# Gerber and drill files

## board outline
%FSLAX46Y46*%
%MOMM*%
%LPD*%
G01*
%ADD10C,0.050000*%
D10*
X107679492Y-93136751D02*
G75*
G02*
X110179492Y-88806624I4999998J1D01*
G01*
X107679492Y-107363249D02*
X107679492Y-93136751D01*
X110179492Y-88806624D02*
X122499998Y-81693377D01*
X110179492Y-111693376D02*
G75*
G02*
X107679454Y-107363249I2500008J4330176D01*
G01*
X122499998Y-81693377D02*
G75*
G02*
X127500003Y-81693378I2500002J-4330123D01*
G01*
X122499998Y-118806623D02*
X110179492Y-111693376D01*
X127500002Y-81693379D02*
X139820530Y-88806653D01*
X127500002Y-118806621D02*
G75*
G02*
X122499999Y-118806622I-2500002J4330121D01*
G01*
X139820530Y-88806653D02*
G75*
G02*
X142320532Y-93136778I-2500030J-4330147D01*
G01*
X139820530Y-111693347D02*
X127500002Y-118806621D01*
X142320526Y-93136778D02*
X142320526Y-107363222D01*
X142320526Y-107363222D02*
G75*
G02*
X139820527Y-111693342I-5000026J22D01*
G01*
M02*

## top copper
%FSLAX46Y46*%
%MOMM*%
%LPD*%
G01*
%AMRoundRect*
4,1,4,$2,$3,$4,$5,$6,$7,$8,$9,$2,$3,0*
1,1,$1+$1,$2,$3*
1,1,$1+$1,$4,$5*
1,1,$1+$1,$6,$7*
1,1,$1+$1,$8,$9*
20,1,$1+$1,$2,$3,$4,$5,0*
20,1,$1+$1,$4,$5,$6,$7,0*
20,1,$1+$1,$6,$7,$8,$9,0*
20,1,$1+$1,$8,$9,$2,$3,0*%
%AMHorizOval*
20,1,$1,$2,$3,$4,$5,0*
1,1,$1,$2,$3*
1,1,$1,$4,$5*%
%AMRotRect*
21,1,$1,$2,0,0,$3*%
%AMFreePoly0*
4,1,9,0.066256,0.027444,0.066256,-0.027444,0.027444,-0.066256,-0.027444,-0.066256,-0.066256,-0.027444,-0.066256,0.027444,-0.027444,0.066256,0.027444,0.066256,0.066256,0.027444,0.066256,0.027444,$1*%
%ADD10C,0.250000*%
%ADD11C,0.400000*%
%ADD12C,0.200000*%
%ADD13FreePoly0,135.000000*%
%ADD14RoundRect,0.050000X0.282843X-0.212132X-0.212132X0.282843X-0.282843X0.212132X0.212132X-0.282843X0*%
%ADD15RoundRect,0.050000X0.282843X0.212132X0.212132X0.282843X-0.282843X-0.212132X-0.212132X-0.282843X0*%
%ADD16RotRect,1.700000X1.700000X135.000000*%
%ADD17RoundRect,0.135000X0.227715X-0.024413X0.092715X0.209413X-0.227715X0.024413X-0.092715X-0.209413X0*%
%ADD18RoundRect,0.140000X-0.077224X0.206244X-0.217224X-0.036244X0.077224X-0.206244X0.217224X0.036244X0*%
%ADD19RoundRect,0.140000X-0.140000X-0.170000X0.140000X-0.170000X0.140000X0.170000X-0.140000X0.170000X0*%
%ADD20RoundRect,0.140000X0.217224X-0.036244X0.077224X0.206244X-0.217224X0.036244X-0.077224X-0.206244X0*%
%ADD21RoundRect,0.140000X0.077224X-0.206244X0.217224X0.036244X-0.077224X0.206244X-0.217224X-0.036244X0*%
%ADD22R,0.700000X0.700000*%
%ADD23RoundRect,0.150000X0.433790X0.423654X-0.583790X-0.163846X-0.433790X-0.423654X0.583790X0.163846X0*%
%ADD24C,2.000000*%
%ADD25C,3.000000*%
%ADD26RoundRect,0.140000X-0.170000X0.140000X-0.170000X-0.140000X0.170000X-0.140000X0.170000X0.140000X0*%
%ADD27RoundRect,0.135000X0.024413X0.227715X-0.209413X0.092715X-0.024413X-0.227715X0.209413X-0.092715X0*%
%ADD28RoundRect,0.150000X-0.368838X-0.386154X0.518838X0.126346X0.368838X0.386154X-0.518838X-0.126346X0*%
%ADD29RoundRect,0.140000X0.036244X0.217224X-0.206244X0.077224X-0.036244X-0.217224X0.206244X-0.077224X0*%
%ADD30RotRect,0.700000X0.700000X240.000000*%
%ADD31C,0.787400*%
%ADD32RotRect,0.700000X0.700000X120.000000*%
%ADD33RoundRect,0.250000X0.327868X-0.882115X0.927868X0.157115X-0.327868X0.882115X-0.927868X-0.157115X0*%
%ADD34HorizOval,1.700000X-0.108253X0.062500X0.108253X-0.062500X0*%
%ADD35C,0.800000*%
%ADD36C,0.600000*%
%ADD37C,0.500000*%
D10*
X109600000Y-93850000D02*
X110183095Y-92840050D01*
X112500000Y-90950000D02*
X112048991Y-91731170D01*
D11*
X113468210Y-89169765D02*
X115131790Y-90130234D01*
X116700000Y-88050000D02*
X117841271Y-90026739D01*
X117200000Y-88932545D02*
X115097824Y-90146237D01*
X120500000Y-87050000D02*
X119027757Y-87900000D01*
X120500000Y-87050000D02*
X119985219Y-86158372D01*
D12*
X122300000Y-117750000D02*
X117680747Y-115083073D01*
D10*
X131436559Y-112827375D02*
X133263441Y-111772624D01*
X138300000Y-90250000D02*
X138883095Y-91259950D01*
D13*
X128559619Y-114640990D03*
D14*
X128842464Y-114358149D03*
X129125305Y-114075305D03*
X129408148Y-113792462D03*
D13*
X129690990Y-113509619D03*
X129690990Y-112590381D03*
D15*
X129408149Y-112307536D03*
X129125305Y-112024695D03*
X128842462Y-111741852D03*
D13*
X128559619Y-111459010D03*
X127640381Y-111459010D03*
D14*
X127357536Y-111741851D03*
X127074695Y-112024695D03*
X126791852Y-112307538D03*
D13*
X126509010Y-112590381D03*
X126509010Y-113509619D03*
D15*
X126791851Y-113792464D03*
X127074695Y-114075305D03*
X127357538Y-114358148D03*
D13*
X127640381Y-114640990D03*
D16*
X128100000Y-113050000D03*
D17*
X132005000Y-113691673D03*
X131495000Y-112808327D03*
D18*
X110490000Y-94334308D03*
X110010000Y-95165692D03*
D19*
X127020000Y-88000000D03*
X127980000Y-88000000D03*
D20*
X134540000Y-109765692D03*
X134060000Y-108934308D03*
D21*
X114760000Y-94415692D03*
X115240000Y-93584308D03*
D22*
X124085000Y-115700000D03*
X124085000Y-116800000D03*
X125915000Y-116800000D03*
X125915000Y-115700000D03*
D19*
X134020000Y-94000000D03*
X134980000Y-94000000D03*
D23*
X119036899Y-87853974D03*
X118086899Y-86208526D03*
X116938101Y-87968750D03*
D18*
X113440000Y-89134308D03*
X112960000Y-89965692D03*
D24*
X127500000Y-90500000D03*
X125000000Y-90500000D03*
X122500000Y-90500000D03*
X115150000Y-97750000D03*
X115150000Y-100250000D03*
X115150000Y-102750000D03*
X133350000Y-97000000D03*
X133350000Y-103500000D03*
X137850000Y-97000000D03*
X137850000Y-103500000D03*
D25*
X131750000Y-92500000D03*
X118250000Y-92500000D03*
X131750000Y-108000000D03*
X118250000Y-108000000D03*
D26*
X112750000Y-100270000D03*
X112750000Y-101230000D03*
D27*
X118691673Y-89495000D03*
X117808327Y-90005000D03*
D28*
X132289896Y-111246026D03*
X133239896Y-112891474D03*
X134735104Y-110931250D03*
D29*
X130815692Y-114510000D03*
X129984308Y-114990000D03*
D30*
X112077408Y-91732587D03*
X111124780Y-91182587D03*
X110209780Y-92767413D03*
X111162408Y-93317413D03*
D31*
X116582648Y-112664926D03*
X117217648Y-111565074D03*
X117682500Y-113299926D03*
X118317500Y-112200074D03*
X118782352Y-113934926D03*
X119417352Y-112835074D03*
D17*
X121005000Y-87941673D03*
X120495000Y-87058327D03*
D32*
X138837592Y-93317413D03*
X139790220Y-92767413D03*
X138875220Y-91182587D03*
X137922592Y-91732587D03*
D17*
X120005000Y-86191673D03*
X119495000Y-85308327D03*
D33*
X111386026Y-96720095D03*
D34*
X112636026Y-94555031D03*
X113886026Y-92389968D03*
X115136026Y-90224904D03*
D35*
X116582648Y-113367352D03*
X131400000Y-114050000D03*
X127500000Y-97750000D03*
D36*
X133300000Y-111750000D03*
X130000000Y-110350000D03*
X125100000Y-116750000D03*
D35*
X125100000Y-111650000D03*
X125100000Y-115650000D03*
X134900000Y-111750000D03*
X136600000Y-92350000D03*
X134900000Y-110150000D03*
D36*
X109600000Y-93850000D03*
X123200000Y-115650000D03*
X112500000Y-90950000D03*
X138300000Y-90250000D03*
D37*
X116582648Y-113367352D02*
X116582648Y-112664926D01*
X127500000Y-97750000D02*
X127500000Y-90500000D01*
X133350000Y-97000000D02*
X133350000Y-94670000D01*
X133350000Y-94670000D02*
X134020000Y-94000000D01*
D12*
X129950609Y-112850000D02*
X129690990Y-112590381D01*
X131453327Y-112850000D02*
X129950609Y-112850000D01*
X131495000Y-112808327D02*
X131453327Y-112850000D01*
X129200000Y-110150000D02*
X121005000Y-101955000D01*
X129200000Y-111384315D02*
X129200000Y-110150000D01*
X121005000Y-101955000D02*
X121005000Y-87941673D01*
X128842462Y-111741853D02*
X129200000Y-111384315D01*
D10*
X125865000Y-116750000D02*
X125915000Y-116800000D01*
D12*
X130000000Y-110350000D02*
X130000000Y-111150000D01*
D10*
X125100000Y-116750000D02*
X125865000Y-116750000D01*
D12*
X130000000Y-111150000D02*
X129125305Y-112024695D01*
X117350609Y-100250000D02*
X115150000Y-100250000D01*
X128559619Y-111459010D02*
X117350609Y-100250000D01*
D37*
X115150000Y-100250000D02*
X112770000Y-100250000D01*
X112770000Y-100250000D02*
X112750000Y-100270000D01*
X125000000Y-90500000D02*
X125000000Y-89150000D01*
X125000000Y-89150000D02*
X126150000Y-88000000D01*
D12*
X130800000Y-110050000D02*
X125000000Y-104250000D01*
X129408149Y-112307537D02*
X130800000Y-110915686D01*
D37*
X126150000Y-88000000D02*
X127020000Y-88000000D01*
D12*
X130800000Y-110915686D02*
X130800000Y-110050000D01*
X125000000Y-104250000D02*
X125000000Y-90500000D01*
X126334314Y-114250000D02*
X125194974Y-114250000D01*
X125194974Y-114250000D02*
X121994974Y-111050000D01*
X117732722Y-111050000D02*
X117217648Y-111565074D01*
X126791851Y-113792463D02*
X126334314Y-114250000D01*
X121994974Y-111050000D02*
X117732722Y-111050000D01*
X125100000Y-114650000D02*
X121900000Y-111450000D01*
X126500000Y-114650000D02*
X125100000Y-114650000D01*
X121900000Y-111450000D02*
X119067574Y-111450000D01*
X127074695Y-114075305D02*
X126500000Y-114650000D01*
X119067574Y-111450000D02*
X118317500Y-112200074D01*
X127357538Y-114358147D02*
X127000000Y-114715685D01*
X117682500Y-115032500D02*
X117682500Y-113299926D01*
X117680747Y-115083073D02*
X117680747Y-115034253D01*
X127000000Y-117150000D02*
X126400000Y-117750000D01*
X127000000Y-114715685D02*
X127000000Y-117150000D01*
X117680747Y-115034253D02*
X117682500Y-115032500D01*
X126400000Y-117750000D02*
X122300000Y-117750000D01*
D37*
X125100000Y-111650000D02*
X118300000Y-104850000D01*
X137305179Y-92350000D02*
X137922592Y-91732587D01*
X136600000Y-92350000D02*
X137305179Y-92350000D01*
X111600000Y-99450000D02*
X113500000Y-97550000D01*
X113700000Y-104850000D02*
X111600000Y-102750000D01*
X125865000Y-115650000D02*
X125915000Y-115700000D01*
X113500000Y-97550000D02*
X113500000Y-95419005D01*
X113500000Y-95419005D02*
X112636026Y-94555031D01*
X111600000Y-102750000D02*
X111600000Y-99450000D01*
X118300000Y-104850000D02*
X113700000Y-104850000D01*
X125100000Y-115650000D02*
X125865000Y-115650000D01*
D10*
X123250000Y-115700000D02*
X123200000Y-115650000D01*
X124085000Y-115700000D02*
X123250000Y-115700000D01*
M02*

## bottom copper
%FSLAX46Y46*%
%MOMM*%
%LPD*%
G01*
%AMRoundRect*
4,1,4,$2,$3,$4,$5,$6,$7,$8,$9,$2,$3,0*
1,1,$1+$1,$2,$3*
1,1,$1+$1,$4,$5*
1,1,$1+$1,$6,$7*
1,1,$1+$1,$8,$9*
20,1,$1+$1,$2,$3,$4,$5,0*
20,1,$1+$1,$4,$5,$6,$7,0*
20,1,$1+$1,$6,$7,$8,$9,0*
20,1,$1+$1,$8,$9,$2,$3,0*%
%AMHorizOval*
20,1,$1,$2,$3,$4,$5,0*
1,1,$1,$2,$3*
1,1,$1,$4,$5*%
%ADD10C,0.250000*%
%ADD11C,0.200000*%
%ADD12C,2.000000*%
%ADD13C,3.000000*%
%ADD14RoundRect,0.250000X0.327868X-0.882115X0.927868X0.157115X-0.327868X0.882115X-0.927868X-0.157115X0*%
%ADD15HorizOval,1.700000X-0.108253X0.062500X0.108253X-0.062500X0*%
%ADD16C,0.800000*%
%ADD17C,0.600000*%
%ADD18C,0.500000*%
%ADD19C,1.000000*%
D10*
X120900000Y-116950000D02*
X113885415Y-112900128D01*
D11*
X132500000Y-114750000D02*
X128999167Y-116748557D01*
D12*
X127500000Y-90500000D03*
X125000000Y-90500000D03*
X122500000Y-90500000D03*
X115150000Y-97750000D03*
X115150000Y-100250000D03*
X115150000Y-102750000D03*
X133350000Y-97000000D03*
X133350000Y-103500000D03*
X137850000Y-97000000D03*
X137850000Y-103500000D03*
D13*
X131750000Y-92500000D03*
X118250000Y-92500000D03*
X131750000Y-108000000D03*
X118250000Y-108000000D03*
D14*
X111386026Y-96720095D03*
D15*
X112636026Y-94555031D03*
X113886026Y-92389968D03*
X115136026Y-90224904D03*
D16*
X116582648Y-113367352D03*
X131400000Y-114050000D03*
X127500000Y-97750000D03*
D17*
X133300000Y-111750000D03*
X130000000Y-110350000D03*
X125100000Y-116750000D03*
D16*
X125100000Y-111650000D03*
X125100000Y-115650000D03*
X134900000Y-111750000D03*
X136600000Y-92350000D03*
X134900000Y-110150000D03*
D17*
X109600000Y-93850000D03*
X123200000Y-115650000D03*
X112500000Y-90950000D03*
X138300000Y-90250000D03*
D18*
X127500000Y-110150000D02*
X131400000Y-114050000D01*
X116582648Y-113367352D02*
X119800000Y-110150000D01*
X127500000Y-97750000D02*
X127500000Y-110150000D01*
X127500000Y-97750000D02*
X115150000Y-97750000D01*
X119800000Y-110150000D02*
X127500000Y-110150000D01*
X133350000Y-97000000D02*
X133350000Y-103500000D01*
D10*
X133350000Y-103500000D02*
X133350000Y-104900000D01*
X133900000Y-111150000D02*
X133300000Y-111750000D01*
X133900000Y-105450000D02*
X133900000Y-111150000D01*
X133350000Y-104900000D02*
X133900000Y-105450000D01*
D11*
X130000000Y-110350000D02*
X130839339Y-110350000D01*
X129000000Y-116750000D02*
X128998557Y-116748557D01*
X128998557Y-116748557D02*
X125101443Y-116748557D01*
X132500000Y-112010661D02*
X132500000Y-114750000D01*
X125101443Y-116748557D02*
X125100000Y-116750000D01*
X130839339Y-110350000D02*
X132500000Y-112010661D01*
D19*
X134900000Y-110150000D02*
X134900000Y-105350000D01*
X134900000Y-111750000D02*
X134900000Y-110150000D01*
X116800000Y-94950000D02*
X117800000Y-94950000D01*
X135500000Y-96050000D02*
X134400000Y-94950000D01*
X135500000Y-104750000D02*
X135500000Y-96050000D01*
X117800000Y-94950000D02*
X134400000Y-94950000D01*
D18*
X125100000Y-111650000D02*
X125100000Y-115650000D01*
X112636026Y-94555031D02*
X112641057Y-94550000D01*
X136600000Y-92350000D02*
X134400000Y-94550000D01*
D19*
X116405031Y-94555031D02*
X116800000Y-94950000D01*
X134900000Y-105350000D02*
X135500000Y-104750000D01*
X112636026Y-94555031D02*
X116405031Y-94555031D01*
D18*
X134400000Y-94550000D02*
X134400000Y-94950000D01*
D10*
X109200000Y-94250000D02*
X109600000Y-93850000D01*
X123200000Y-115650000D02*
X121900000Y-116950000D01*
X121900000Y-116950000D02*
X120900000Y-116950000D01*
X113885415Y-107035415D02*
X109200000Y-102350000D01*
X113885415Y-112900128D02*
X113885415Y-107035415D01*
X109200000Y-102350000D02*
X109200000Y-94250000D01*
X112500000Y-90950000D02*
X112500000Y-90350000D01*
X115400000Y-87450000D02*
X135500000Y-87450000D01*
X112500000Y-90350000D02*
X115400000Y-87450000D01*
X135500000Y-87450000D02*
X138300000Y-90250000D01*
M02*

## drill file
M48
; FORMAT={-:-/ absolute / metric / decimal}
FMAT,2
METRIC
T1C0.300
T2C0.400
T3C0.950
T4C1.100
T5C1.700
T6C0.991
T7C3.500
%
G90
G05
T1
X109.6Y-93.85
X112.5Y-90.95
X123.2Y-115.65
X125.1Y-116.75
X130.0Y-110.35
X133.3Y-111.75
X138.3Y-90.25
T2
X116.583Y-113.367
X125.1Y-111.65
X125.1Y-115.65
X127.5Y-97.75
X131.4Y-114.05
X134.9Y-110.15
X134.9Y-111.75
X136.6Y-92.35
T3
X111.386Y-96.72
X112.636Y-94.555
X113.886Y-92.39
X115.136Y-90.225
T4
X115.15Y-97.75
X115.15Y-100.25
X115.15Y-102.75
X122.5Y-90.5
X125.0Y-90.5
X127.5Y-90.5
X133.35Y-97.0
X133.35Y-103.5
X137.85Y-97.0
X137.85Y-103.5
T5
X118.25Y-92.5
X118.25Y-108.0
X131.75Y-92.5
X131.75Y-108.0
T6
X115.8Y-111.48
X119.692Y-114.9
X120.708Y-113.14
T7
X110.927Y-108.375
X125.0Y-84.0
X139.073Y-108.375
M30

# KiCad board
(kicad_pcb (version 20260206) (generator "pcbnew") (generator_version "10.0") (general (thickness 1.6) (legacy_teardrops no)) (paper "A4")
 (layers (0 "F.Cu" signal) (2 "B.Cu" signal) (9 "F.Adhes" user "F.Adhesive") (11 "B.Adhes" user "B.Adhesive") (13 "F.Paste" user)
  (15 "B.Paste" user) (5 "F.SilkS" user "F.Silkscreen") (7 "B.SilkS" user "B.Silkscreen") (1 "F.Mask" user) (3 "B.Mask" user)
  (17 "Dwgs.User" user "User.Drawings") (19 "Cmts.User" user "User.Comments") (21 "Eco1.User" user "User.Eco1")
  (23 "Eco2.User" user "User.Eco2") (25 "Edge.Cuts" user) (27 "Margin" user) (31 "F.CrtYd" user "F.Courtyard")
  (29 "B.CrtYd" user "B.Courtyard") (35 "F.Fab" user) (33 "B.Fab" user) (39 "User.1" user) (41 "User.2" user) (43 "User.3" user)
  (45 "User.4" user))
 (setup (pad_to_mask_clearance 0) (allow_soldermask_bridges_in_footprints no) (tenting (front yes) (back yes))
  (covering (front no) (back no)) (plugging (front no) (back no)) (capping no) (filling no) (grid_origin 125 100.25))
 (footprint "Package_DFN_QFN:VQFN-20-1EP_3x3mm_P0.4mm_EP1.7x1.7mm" (layer "F.Cu") (at 128.1 113.05 135)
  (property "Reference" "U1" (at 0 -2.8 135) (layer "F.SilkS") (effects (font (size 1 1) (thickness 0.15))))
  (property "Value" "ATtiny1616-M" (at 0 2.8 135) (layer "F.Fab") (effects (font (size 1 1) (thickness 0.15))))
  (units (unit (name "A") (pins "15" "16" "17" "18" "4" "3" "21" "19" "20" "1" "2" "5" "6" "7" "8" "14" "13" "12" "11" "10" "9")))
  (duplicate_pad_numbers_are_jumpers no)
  (pad "" smd roundrect (at -0.425 -0.425 135) (size 0.69 0.69) (layers "F.Paste") (roundrect_rratio 0.25))
  (pad "" smd roundrect (at -0.425 0.425 135) (size 0.69 0.69) (layers "F.Paste") (roundrect_rratio 0.25))
  (pad "" smd roundrect (at 0.425 -0.425 135) (size 0.69 0.69) (layers "F.Paste") (roundrect_rratio 0.25))
  (pad "" smd roundrect (at 0.425 0.425 135) (size 0.69 0.69) (layers "F.Paste") (roundrect_rratio 0.25))
  (pad "1" smd custom (at -1.45 -0.8 135) (size 0.143431 0.143431) (layers "F.Cu" "F.Mask" "F.Paste") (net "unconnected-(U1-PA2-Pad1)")
   (options (clearance outline) (anchor circle)) (primitives))
  (pad "2" smd roundrect (at -1.450002 -0.4 135) (size 0.8 0.2) (layers "F.Cu" "F.Mask" "F.Paste") (roundrect_rratio 0.25)
   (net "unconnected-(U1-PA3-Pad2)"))
  (pad "3" smd roundrect (at -1.45 0 135) (size 0.8 0.2) (layers "F.Cu" "F.Mask" "F.Paste") (roundrect_rratio 0.25) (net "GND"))
  (pad "4" smd roundrect (at -1.45 0.4 135) (size 0.8 0.2) (layers "F.Cu" "F.Mask" "F.Paste") (roundrect_rratio 0.25) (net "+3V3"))
  (pad "5" smd custom (at -1.45 0.8 135) (size 0.143431 0.143431) (layers "F.Cu" "F.Mask" "F.Paste") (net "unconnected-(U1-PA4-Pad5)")
   (options (clearance outline) (anchor circle)) (primitives))
  (pad "6" smd custom (at -0.8 1.45 135) (size 0.143431 0.143431) (layers "F.Cu" "F.Mask" "F.Paste") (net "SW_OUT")
   (options (clearance outline) (anchor circle)) (primitives))
  (pad "7" smd roundrect (at -0.4 1.450002 135) (size 0.2 0.8) (layers "F.Cu" "F.Mask" "F.Paste") (roundrect_rratio 0.25) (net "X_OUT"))
  (pad "8" smd roundrect (at 0 1.45 135) (size 0.2 0.8) (layers "F.Cu" "F.Mask" "F.Paste") (roundrect_rratio 0.25) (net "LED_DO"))
  (pad "9" smd roundrect (at 0.4 1.45 135) (size 0.2 0.8) (layers "F.Cu" "F.Mask" "F.Paste") (roundrect_rratio 0.25) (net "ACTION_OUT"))
  (pad "10" smd custom (at 0.8 1.45 135) (size 0.143431 0.143431) (layers "F.Cu" "F.Mask" "F.Paste") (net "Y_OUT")
   (options (clearance outline) (anchor circle)) (primitives))
  (pad "11" smd custom (at 1.45 0.8 135) (size 0.143431 0.143431) (layers "F.Cu" "F.Mask" "F.Paste") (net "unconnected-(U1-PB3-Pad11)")
   (options (clearance outline) (anchor circle)) (primitives))
  (pad "12" smd roundrect (at 1.450002 0.4 135) (size 0.8 0.2) (layers "F.Cu" "F.Mask" "F.Paste") (roundrect_rratio 0.25)
   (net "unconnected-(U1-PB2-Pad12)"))
  (pad "13" smd roundrect (at 1.45 0 135) (size 0.8 0.2) (layers "F.Cu" "F.Mask" "F.Paste") (roundrect_rratio 0.25)
   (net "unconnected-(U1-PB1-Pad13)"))
  (pad "14" smd roundrect (at 1.45 -0.4 135) (size 0.8 0.2) (layers "F.Cu" "F.Mask" "F.Paste") (roundrect_rratio 0.25)
   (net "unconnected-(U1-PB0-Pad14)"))
  (pad "15" smd custom (at 1.45 -0.8 135) (size 0.143431 0.143431) (layers "F.Cu" "F.Mask" "F.Paste") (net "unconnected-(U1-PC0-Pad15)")
   (options (clearance outline) (anchor circle)) (primitives))
  (pad "16" smd custom (at 0.8 -1.45 135) (size 0.143431 0.143431) (layers "F.Cu" "F.Mask" "F.Paste") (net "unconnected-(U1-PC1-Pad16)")
   (options (clearance outline) (anchor circle)) (primitives))
  (pad "17" smd roundrect (at 0.4 -1.450002 135) (size 0.2 0.8) (layers "F.Cu" "F.Mask" "F.Paste") (roundrect_rratio 0.25) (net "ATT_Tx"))
  (pad "18" smd roundrect (at 0 -1.45 135) (size 0.2 0.8) (layers "F.Cu" "F.Mask" "F.Paste") (roundrect_rratio 0.25) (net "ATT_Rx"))
  (pad "19" smd roundrect (at -0.4 -1.45 135) (size 0.2 0.8) (layers "F.Cu" "F.Mask" "F.Paste") (roundrect_rratio 0.25) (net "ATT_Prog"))
  (pad "20" smd custom (at -0.8 -1.45 135) (size 0.143431 0.143431) (layers "F.Cu" "F.Mask" "F.Paste") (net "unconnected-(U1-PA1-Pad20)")
   (options (clearance outline) (anchor circle)) (primitives))
  (pad "21" smd rect (at 0 0 135) (size 1.7 1.7) (layers "F.Cu" "F.Mask") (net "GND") (zone_connect 2)))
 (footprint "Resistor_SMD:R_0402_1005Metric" (layer "F.Cu") (at 131.75 113.25 120)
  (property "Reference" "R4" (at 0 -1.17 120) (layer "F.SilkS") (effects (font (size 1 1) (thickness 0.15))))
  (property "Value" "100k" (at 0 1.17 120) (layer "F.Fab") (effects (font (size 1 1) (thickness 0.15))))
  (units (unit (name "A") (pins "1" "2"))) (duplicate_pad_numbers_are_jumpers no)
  (pad "1" smd roundrect (at -0.51 0 120) (size 0.54 0.64) (layers "F.Cu" "F.Mask" "F.Paste") (roundrect_rratio 0.25) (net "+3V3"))
  (pad "2" smd roundrect (at 0.51 0 120) (size 0.54 0.64) (layers "F.Cu" "F.Mask" "F.Paste") (roundrect_rratio 0.25) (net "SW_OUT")))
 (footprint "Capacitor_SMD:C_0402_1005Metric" (layer "F.Cu") (at 110.25 94.75 -120)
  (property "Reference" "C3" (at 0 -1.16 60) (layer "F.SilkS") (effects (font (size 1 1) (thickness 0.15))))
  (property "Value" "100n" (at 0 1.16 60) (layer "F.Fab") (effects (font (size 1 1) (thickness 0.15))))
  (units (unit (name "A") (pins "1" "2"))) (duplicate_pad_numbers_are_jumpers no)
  (pad "1" smd roundrect (at -0.48 0 240) (size 0.56 0.62) (layers "F.Cu" "F.Mask" "F.Paste") (roundrect_rratio 0.25) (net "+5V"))
  (pad "2" smd roundrect (at 0.48 0 240) (size 0.56 0.62) (layers "F.Cu" "F.Mask" "F.Paste") (roundrect_rratio 0.25) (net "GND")))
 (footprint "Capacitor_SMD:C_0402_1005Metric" (layer "F.Cu") (at 127.5 88)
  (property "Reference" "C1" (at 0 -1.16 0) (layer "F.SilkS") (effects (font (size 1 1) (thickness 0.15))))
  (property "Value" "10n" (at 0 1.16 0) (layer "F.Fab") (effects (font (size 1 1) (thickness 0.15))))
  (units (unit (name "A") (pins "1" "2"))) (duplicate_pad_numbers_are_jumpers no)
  (pad "1" smd roundrect (at -0.48 0) (size 0.56 0.62) (layers "F.Cu" "F.Mask" "F.Paste") (roundrect_rratio 0.25) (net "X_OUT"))
  (pad "2" smd roundrect (at 0.48 0) (size 0.56 0.62) (layers "F.Cu" "F.Mask" "F.Paste") (roundrect_rratio 0.25) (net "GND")))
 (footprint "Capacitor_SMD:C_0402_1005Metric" (layer "F.Cu") (at 134.3 109.35 120)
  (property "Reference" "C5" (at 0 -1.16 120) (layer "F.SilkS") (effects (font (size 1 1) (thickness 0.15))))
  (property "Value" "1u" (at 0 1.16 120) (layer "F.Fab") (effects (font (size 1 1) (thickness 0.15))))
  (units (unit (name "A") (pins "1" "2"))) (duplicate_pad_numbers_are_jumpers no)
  (pad "1" smd roundrect (at -0.48 0 120) (size 0.56 0.62) (layers "F.Cu" "F.Mask" "F.Paste") (roundrect_rratio 0.25) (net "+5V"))
  (pad "2" smd roundrect (at 0.48 0 120) (size 0.56 0.62) (layers "F.Cu" "F.Mask" "F.Paste") (roundrect_rratio 0.25) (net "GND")))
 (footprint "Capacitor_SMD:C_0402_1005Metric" (layer "F.Cu") (at 115 94 60)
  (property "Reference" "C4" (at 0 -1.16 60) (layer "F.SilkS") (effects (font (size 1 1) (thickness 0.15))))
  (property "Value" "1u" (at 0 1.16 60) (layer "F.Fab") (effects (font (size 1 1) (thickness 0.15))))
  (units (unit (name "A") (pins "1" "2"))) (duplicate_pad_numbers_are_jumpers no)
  (pad "1" smd roundrect (at -0.48 0 60) (size 0.56 0.62) (layers "F.Cu" "F.Mask" "F.Paste") (roundrect_rratio 0.25) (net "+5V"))
  (pad "2" smd roundrect (at 0.48 0 60) (size 0.56 0.62) (layers "F.Cu" "F.Mask" "F.Paste") (roundrect_rratio 0.25) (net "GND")))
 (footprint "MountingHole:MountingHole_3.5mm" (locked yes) (layer "F.Cu") (at 110.927087 108.375)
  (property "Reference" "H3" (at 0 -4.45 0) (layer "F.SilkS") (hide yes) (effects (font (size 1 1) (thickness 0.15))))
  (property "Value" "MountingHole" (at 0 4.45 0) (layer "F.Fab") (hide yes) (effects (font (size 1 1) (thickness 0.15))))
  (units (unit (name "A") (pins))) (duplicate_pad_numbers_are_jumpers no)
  (pad "" np_thru_hole circle (at 0 0) (size 3.5 3.5) (drill 3.5) (layers "*.Cu" "*.Mask")))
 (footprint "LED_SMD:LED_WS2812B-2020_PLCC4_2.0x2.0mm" (layer "F.Cu") (at 125 116.25)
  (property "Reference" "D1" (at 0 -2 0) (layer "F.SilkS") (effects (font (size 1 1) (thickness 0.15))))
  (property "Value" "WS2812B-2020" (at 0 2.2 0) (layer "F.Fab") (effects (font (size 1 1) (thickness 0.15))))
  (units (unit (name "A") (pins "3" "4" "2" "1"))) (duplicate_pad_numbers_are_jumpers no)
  (pad "1" smd rect (at -0.915 -0.55) (size 0.7 0.7) (layers "F.Cu" "F.Mask" "F.Paste") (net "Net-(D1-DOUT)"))
  (pad "2" smd rect (at -0.915 0.55) (size 0.7 0.7) (layers "F.Cu" "F.Mask" "F.Paste") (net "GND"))
  (pad "3" smd rect (at 0.915 0.55) (size 0.7 0.7) (layers "F.Cu" "F.Mask" "F.Paste") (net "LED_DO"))
  (pad "4" smd rect (at 0.915 -0.55) (size 0.7 0.7) (layers "F.Cu" "F.Mask" "F.Paste") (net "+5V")))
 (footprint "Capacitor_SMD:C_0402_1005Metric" (layer "F.Cu") (at 134.5 94)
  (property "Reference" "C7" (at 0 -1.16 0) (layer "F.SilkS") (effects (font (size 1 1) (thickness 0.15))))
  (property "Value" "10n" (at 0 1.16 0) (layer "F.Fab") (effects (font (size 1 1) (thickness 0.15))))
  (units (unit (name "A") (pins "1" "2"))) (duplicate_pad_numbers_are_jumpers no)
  (pad "1" smd roundrect (at -0.48 0) (size 0.56 0.62) (layers "F.Cu" "F.Mask" "F.Paste") (roundrect_rratio 0.25) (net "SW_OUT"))
  (pad "2" smd roundrect (at 0.48 0) (size 0.56 0.62) (layers "F.Cu" "F.Mask" "F.Paste") (roundrect_rratio 0.25) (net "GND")))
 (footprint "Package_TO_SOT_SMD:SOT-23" (layer "F.Cu") (at 117.75 87.5 -150)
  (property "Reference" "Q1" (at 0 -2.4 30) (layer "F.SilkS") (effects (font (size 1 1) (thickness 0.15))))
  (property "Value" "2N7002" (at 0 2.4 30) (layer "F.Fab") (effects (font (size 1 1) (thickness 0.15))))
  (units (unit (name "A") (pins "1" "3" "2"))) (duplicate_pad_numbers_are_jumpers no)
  (pad "1" smd roundrect (at -0.9375 -0.95 210) (size 1.475 0.6) (layers "F.Cu" "F.Mask" "F.Paste") (roundrect_rratio 0.25)
   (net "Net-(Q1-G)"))
  (pad "2" smd roundrect (at -0.9375 0.95 210) (size 1.475 0.6) (layers "F.Cu" "F.Mask" "F.Paste") (roundrect_rratio 0.25) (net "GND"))
  (pad "3" smd roundrect (at 0.9375 0 210) (size 1.475 0.6) (layers "F.Cu" "F.Mask" "F.Paste") (roundrect_rratio 0.25) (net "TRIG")))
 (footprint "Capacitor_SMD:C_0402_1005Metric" (layer "F.Cu") (at 113.2 89.55 -120)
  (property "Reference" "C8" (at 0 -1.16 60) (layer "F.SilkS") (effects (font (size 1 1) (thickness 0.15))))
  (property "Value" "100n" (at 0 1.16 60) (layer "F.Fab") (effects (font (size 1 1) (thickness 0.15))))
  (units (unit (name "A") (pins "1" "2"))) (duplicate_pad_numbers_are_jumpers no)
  (pad "1" smd roundrect (at -0.48 0 240) (size 0.56 0.62) (layers "F.Cu" "F.Mask" "F.Paste") (roundrect_rratio 0.25) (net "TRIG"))
  (pad "2" smd roundrect (at 0.48 0 240) (size 0.56 0.62) (layers "F.Cu" "F.Mask" "F.Paste") (roundrect_rratio 0.25) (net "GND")))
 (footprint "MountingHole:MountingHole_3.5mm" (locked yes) (layer "F.Cu") (at 125 84)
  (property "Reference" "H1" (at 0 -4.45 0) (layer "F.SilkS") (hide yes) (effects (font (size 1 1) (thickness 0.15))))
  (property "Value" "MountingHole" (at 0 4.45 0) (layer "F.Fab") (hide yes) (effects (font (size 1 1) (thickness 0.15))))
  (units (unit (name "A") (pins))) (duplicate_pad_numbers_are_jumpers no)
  (pad "" np_thru_hole circle (at 0 0) (size 3.5 3.5) (drill 3.5) (layers "*.Cu" "*.Mask")))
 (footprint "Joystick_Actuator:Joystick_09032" (layer "F.Cu") (at 125 100.25 -90)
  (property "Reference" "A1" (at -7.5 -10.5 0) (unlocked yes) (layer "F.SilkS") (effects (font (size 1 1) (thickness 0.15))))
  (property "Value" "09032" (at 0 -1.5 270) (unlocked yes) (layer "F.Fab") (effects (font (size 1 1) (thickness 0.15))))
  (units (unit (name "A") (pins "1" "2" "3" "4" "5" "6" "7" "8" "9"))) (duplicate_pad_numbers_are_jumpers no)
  (pad "1" thru_hole circle (at -9.75 -2.5 270) (size 2 2) (drill 1.1) (layers "*.Cu" "*.Mask") (remove_unused_layers no) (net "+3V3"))
  (pad "2" thru_hole circle (at -9.75 0 270) (size 2 2) (drill 1.1) (layers "*.Cu" "*.Mask") (remove_unused_layers no) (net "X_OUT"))
  (pad "3" thru_hole circle (at -9.75 2.5 270) (size 2 2) (drill 1.1) (layers "*.Cu" "*.Mask") (remove_unused_layers no) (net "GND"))
  (pad "4" thru_hole circle (at -2.5 9.85 270) (size 2 2) (drill 1.1) (layers "*.Cu" "*.Mask") (remove_unused_layers no) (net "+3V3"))
  (pad "5" thru_hole circle (at 0 9.85 270) (size 2 2) (drill 1.1) (layers "*.Cu" "*.Mask") (remove_unused_layers no) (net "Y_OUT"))
  (pad "6" thru_hole circle (at 2.5 9.85 270) (size 2 2) (drill 1.1) (layers "*.Cu" "*.Mask") (remove_unused_layers no) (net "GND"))
  (pad "7" thru_hole circle (at -3.25 -8.35 270) (size 2 2) (drill 1.1) (layers "*.Cu" "*.Mask") (remove_unused_layers no) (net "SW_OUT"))
  (pad "7" thru_hole circle (at 3.25 -8.35 270) (size 2 2) (drill 1.1) (layers "*.Cu" "*.Mask") (remove_unused_layers no) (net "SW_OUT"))
  (pad "8" thru_hole circle (at -3.25 -12.85 270) (size 2 2) (drill 1.1) (layers "*.Cu" "*.Mask") (remove_unused_layers no) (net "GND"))
  (pad "8" thru_hole circle (at 3.25 -12.85 270) (size 2 2) (drill 1.1) (layers "*.Cu" "*.Mask") (remove_unused_layers no) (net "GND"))
  (pad "9" thru_hole circle (at -7.75 -6.75 270) (size 3 3) (drill 1.7) (layers "*.Cu" "*.Mask") (remove_unused_layers no) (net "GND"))
  (pad "9" thru_hole circle (at -7.75 6.75 270) (size 3 3) (drill 1.7) (layers "*.Cu" "*.Mask") (remove_unused_layers no) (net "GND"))
  (pad "9" thru_hole circle (at 7.75 -6.75 270) (size 3 3) (drill 1.7) (layers "*.Cu" "*.Mask") (remove_unused_layers no) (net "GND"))
  (pad "9" thru_hole circle (at 7.75 6.75 270) (size 3 3) (drill 1.7) (layers "*.Cu" "*.Mask") (remove_unused_layers no) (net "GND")))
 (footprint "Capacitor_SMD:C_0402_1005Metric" (layer "F.Cu") (at 112.75 100.75 -90)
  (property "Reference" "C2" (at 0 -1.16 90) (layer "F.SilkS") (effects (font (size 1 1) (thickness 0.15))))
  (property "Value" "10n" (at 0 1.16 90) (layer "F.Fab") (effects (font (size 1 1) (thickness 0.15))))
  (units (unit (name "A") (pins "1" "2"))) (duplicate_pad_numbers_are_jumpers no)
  (pad "1" smd roundrect (at -0.48 0 270) (size 0.56 0.62) (layers "F.Cu" "F.Mask" "F.Paste") (roundrect_rratio 0.25) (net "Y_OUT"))
  (pad "2" smd roundrect (at 0.48 0 270) (size 0.56 0.62) (layers "F.Cu" "F.Mask" "F.Paste") (roundrect_rratio 0.25) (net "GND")))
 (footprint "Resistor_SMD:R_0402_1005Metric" (layer "F.Cu") (at 118.25 89.75 -150)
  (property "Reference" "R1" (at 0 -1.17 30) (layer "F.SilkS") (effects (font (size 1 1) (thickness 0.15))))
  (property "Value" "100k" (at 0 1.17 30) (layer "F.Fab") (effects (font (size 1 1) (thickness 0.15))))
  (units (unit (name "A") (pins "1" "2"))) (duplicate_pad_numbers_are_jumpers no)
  (pad "1" smd roundrect (at -0.51 0 210) (size 0.54 0.64) (layers "F.Cu" "F.Mask" "F.Paste") (roundrect_rratio 0.25) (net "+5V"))
  (pad "2" smd roundrect (at 0.51 0 210) (size 0.54 0.64) (layers "F.Cu" "F.Mask" "F.Paste") (roundrect_rratio 0.25) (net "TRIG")))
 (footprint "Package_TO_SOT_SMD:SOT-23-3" (layer "F.Cu") (at 133.75 111.5 30)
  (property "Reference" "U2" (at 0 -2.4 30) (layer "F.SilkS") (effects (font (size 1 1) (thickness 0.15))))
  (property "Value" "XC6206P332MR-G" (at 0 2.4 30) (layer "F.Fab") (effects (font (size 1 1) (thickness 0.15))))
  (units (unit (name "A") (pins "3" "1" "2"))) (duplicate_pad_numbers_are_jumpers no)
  (pad "1" smd roundrect (at -1.1375 -0.95 30) (size 1.325 0.6) (layers "F.Cu" "F.Mask" "F.Paste") (roundrect_rratio 0.25) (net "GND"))
  (pad "2" smd roundrect (at -1.1375 0.95 30) (size 1.325 0.6) (layers "F.Cu" "F.Mask" "F.Paste") (roundrect_rratio 0.25) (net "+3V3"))
  (pad "3" smd roundrect (at 1.1375 0 30) (size 1.325 0.6) (layers "F.Cu" "F.Mask" "F.Paste") (roundrect_rratio 0.25) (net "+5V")))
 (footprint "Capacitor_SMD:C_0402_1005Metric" (layer "F.Cu") (at 130.4 114.75 -150)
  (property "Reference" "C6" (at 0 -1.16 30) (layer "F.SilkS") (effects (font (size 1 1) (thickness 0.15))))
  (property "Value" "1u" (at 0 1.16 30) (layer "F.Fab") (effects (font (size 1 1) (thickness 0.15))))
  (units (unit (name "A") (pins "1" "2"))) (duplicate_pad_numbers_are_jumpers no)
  (pad "1" smd roundrect (at -0.48 0 210) (size 0.56 0.62) (layers "F.Cu" "F.Mask" "F.Paste") (roundrect_rratio 0.25) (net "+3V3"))
  (pad "2" smd roundrect (at 0.48 0 210) (size 0.56 0.62) (layers "F.Cu" "F.Mask" "F.Paste") (roundrect_rratio 0.25) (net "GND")))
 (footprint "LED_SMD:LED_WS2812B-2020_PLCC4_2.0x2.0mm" (layer "F.Cu") (at 111.143594 92.25 -120)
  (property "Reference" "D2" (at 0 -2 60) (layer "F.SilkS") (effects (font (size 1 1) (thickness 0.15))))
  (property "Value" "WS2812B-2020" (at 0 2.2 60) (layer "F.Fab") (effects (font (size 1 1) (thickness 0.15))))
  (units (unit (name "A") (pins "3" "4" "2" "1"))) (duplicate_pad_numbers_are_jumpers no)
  (pad "1" smd rect (at -0.915 -0.55 240) (size 0.7 0.7) (layers "F.Cu" "F.Mask" "F.Paste") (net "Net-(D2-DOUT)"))
  (pad "2" smd rect (at -0.915 0.55 240) (size 0.7 0.7) (layers "F.Cu" "F.Mask" "F.Paste") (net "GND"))
  (pad "3" smd rect (at 0.915 0.55 240) (size 0.7 0.7) (layers "F.Cu" "F.Mask" "F.Paste") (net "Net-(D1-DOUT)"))
  (pad "4" smd rect (at 0.915 -0.55 240) (size 0.7 0.7) (layers "F.Cu" "F.Mask" "F.Paste") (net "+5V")))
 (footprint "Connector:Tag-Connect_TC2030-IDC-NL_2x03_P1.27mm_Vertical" (layer "F.Cu") (at 118 112.75 -30)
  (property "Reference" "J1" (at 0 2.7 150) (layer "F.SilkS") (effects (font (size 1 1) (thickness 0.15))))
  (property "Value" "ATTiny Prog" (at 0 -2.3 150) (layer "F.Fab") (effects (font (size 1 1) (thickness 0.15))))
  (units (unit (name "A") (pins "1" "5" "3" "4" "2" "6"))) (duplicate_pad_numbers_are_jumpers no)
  (pad "" np_thru_hole circle (at -2.54 0 330) (size 0.9906 0.9906) (drill 0.9906) (layers "*.Cu" "*.Mask"))
  (pad "" np_thru_hole circle (at 2.540001 -1.016 330) (size 0.9906 0.9906) (drill 0.9906) (layers "*.Cu" "*.Mask"))
  (pad "" np_thru_hole circle (at 2.540001 1.016 330) (size 0.9906 0.9906) (drill 0.9906) (layers "*.Cu" "*.Mask"))
  (pad "1" connect circle (at -1.27 0.635 330) (size 0.7874 0.7874) (layers "F.Cu" "F.Mask") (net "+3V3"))
  (pad "2" connect circle (at -1.27 -0.635 330) (size 0.7874 0.7874) (layers "F.Cu" "F.Mask") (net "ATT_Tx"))
  (pad "3" connect circle (at 0 0.635 330) (size 0.7874 0.7874) (layers "F.Cu" "F.Mask") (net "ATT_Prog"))
  (pad "4" connect circle (at 0 -0.635 330) (size 0.7874 0.7874) (layers "F.Cu" "F.Mask") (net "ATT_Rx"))
  (pad "5" connect circle (at 1.27 0.635 330) (size 0.7874 0.7874) (layers "F.Cu" "F.Mask") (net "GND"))
  (pad "6" connect circle (at 1.27 -0.635 330) (size 0.7874 0.7874) (layers "F.Cu" "F.Mask") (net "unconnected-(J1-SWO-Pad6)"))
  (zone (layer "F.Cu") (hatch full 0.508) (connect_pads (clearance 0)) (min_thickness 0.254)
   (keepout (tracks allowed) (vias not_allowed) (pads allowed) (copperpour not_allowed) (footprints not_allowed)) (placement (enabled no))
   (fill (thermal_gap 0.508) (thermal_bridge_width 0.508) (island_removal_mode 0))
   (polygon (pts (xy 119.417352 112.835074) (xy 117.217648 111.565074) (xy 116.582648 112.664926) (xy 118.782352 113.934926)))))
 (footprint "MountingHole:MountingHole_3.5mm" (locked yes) (layer "F.Cu") (at 139.072913 108.375)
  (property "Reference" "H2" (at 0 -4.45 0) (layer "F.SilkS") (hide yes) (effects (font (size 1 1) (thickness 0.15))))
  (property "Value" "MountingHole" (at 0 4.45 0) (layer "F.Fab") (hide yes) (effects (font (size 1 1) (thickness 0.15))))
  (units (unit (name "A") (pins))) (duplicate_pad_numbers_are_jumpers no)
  (pad "" np_thru_hole circle (at 0 0) (size 3.5 3.5) (drill 3.5) (layers "*.Cu" "*.Mask")))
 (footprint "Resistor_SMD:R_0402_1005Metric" (layer "F.Cu") (at 120.75 87.5 120)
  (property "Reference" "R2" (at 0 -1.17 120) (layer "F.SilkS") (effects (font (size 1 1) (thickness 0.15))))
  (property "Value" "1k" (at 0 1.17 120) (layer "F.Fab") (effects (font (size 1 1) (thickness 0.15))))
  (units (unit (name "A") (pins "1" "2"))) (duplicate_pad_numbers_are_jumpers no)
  (pad "1" smd roundrect (at -0.51 0 120) (size 0.54 0.64) (layers "F.Cu" "F.Mask" "F.Paste") (roundrect_rratio 0.25) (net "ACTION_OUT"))
  (pad "2" smd roundrect (at 0.51 0 120) (size 0.54 0.64) (layers "F.Cu" "F.Mask" "F.Paste") (roundrect_rratio 0.25) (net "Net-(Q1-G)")))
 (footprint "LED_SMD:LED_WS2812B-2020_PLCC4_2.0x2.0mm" (layer "F.Cu") (at 138.856406 92.25 120)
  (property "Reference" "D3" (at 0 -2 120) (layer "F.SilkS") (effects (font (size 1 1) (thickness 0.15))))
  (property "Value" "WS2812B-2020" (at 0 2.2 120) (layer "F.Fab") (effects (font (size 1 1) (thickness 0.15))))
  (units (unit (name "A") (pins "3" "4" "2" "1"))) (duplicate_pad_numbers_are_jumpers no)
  (pad "1" smd rect (at -0.915 -0.55 120) (size 0.7 0.7) (layers "F.Cu" "F.Mask" "F.Paste") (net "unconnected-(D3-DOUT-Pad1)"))
  (pad "2" smd rect (at -0.915 0.55 120) (size 0.7 0.7) (layers "F.Cu" "F.Mask" "F.Paste") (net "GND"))
  (pad "3" smd rect (at 0.915 0.55 120) (size 0.7 0.7) (layers "F.Cu" "F.Mask" "F.Paste") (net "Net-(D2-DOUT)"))
  (pad "4" smd rect (at 0.915 -0.55 120) (size 0.7 0.7) (layers "F.Cu" "F.Mask" "F.Paste") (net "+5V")))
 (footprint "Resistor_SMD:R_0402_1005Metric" (layer "F.Cu") (at 119.75 85.75 120)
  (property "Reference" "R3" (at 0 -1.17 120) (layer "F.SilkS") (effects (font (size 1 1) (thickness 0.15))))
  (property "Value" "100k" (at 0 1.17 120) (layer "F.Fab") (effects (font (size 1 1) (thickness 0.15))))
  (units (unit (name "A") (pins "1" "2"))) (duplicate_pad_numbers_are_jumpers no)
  (pad "1" smd roundrect (at -0.51 0 120) (size 0.54 0.64) (layers "F.Cu" "F.Mask" "F.Paste") (roundrect_rratio 0.25) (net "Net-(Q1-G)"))
  (pad "2" smd roundrect (at 0.51 0 120) (size 0.54 0.64) (layers "F.Cu" "F.Mask" "F.Paste") (roundrect_rratio 0.25) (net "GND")))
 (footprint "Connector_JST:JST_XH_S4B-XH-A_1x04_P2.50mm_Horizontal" (layer "B.Cu") (at 111.386026 96.720095 60)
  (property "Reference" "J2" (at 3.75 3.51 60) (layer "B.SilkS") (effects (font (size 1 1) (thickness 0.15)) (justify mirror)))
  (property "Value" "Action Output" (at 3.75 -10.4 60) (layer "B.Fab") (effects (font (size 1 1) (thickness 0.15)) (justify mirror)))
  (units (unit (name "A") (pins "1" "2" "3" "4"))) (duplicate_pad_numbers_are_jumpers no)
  (pad "1" thru_hole roundrect (at 0 0 60) (size 1.7 1.95) (drill 0.95) (layers "*.Cu" "*.Mask") (remove_unused_layers no)
   (roundrect_rratio 0.147059) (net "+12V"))
  (pad "2" thru_hole oval (at 2.5 0 60) (size 1.7 1.95) (drill 0.95) (layers "*.Cu" "*.Mask") (remove_unused_layers no) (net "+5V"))
  (pad "3" thru_hole oval (at 5 0 60) (size 1.7 1.95) (drill 0.95) (layers "*.Cu" "*.Mask") (remove_unused_layers no) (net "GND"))
  (pad "4" thru_hole oval (at 7.5 0 60) (size 1.7 1.95) (drill 0.95) (layers "*.Cu" "*.Mask") (remove_unused_layers no) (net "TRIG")))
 (gr_line (start 109.6 93.85) (end 110.183095 92.84005) (stroke (width 0.25) (type solid)) (layer "F.Cu") (net "Net-(D1-DOUT)"))
 (gr_line (start 112.5 90.95) (end 112.048991 91.73117) (stroke (width 0.25) (type solid)) (layer "F.Cu") (net "Net-(D2-DOUT)"))
 (gr_line (start 113.46821 89.169765) (end 115.13179 90.130234) (stroke (width 0.4) (type solid)) (layer "F.Cu") (net "TRIG"))
 (gr_line (start 116.7 88.05) (end 117.841271 90.026739) (stroke (width 0.4) (type solid)) (layer "F.Cu") (net "TRIG"))
 (gr_line (start 117.2 88.932545) (end 115.097824 90.146237) (stroke (width 0.4) (type solid)) (layer "F.Cu") (net "TRIG"))
 (gr_line (start 120.5 87.05) (end 119.027757 87.9) (stroke (width 0.4) (type solid)) (layer "F.Cu") (net "Net-(Q1-G)"))
 (gr_line (start 120.5 87.05) (end 119.985219 86.158372) (stroke (width 0.4) (type solid)) (layer "F.Cu") (net "Net-(Q1-G)"))
 (gr_line (start 122.3 117.75) (end 117.680747 115.083073) (stroke (width 0.2) (type solid)) (layer "F.Cu") (net "ATT_Prog"))
 (gr_line (start 131.436559 112.827375) (end 133.263441 111.772624) (stroke (width 0.25) (type solid)) (layer "F.Cu") (net "SW_OUT"))
 (gr_line (start 138.3 90.25) (end 138.883095 91.25995) (stroke (width 0.25) (type solid)) (layer "F.Cu") (net "Net-(D2-DOUT)"))
 (gr_line (start 120.9 116.95) (end 113.885415 112.900128) (stroke (width 0.25) (type solid)) (layer "B.Cu") (net "Net-(D1-DOUT)"))
 (gr_line (start 132.5 114.75) (end 128.999167 116.748557) (stroke (width 0.2) (type solid)) (layer "B.Cu") (net "LED_DO"))
 (gr_arc (start 107.679492 93.136751) (mid 108.349365 90.636751) (end 110.179492 88.806624) (stroke (width 0.05) (type default))
  (layer "Edge.Cuts"))
 (gr_line (start 107.679492 107.363249) (end 107.679492 93.136751) (stroke (width 0.05) (type default)) (layer "Edge.Cuts"))
 (gr_line (start 110.179492 88.806624) (end 122.499998 81.693377) (stroke (width 0.05) (type default)) (layer "Edge.Cuts"))
 (gr_arc (start 110.179492 111.693376) (mid 108.349365 109.863249) (end 107.679492 107.363249) (stroke (width 0.05) (type default))
  (layer "Edge.Cuts"))
 (gr_arc (start 122.499998 81.693377) (mid 125.000001 81.023502) (end 127.500002 81.693379) (stroke (width 0.05) (type default))
  (layer "Edge.Cuts"))
 (gr_line (start 122.499998 118.806623) (end 110.179492 111.693376) (stroke (width 0.05) (type default)) (layer "Edge.Cuts"))
 (gr_line (start 127.500002 81.693379) (end 139.82053 88.806653) (stroke (width 0.05) (type default)) (layer "Edge.Cuts"))
 (gr_arc (start 127.500002 118.806621) (mid 125 119.476496) (end 122.499998 118.806623) (stroke (width 0.05) (type default))
  (layer "Edge.Cuts"))
 (gr_arc (start 139.82053 88.806653) (mid 141.650654 90.63678) (end 142.320526 93.136778) (stroke (width 0.05) (type default))
  (layer "Edge.Cuts"))
 (gr_line (start 139.82053 111.693347) (end 127.500002 118.806621) (stroke (width 0.05) (type default)) (layer "Edge.Cuts"))
 (gr_line (start 142.320526 93.136778) (end 142.320526 107.363222) (stroke (width 0.05) (type default)) (layer "Edge.Cuts"))
 (gr_arc (start 142.320526 107.363222) (mid 141.650648 109.863216) (end 139.82053 111.693347) (stroke (width 0.05) (type default))
  (layer "Edge.Cuts"))
 (segment (start 116.582648 113.367352) (end 116.582648 112.664926) (width 0.5) (layer "F.Cu") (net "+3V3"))
 (segment (start 127.5 97.75) (end 127.5 90.5) (width 0.5) (layer "F.Cu") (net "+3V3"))
 (via (at 116.582648 113.367352) (size 0.8) (drill 0.4) (layers "F.Cu" "B.Cu") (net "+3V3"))
 (via (at 131.4 114.05) (size 0.8) (drill 0.4) (layers "F.Cu" "B.Cu") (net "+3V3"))
 (via (at 127.5 97.75) (size 0.8) (drill 0.4) (layers "F.Cu" "B.Cu") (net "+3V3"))
 (segment (start 127.5 110.15) (end 131.4 114.05) (width 0.5) (layer "B.Cu") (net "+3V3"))
 (segment (start 116.582648 113.367352) (end 119.8 110.15) (width 0.5) (layer "B.Cu") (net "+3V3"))
 (segment (start 127.5 97.75) (end 127.5 110.15) (width 0.5) (layer "B.Cu") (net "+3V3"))
 (segment (start 127.5 97.75) (end 115.15 97.75) (width 0.5) (layer "B.Cu") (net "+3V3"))
 (segment (start 119.8 110.15) (end 127.5 110.15) (width 0.5) (layer "B.Cu") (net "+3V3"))
 (segment (start 133.35 97) (end 133.35 94.67) (width 0.5) (layer "F.Cu") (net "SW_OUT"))
 (segment (start 133.35 94.67) (end 134.02 94) (width 0.5) (layer "F.Cu") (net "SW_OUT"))
 (segment (start 129.950609 112.85) (end 129.69099 112.590381) (width 0.2) (layer "F.Cu") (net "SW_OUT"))
 (segment (start 131.453327 112.85) (end 129.950609 112.85) (width 0.2) (layer "F.Cu") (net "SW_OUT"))
 (segment (start 131.495 112.808327) (end 131.453327 112.85) (width 0.2) (layer "F.Cu") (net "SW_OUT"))
 (via (at 133.3 111.75) (size 0.6) (drill 0.3) (layers "F.Cu" "B.Cu") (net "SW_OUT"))
 (segment (start 133.35 97) (end 133.35 103.5) (width 0.5) (layer "B.Cu") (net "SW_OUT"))
 (segment (start 133.35 103.5) (end 133.35 104.9) (width 0.25) (layer "B.Cu") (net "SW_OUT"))
 (segment (start 133.9 111.15) (end 133.3 111.75) (width 0.25) (layer "B.Cu") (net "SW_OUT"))
 (segment (start 133.9 105.45) (end 133.9 111.15) (width 0.25) (layer "B.Cu") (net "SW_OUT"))
 (segment (start 133.35 104.9) (end 133.9 105.45) (width 0.25) (layer "B.Cu") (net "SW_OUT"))
 (segment (start 129.2 110.15) (end 121.005 101.955) (width 0.2) (layer "F.Cu") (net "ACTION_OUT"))
 (segment (start 129.2 111.384315) (end 129.2 110.15) (width 0.2) (layer "F.Cu") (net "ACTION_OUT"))
 (segment (start 121.005 101.955) (end 121.005 87.941673) (width 0.2) (layer "F.Cu") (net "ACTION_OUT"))
 (segment (start 128.842462 111.741853) (end 129.2 111.384315) (width 0.2) (layer "F.Cu") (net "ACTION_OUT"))
 (segment (start 125.865 116.75) (end 125.915 116.8) (width 0.25) (layer "F.Cu") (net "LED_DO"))
 (segment (start 130 110.35) (end 130 111.15) (width 0.2) (layer "F.Cu") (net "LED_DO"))
 (segment (start 125.1 116.75) (end 125.865 116.75) (width 0.25) (layer "F.Cu") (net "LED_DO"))
 (segment (start 130 111.15) (end 129.125305 112.024695) (width 0.2) (layer "F.Cu") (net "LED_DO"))
 (via (at 130 110.35) (size 0.6) (drill 0.3) (layers "F.Cu" "B.Cu") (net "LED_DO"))
 (via (at 125.1 116.75) (size 0.6) (drill 0.3) (layers "F.Cu" "B.Cu") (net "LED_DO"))
 (segment (start 130 110.35) (end 130.839339 110.35) (width 0.2) (layer "B.Cu") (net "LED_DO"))
 (segment (start 129 116.75) (end 128.998557 116.748557) (width 0.2) (layer "B.Cu") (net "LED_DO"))
 (segment (start 128.998557 116.748557) (end 125.101443 116.748557) (width 0.2) (layer "B.Cu") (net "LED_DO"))
 (segment (start 132.5 112.010661) (end 132.5 114.75) (width 0.2) (layer "B.Cu") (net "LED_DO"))
 (segment (start 125.101443 116.748557) (end 125.1 116.75) (width 0.2) (layer "B.Cu") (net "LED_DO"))
 (segment (start 130.839339 110.35) (end 132.5 112.010661) (width 0.2) (layer "B.Cu") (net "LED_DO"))
 (segment (start 117.350609 100.25) (end 115.15 100.25) (width 0.2) (layer "F.Cu") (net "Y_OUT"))
 (segment (start 128.559619 111.45901) (end 117.350609 100.25) (width 0.2) (layer "F.Cu") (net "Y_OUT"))
 (segment (start 115.15 100.25) (end 112.77 100.25) (width 0.5) (layer "F.Cu") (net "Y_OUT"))
 (segment (start 112.77 100.25) (end 112.75 100.27) (width 0.5) (layer "F.Cu") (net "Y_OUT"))
 (segment (start 125 90.5) (end 125 89.15) (width 0.5) (layer "F.Cu") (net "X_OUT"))
 (segment (start 125 89.15) (end 126.15 88) (width 0.5) (layer "F.Cu") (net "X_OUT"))
 (segment (start 130.8 110.05) (end 125 104.25) (width 0.2) (layer "F.Cu") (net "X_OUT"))
 (segment (start 129.408149 112.307537) (end 130.8 110.915686) (width 0.2) (layer "F.Cu") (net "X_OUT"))
 (segment (start 126.15 88) (end 127.02 88) (width 0.5) (layer "F.Cu") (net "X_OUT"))
 (segment (start 130.8 110.915686) (end 130.8 110.05) (width 0.2) (layer "F.Cu") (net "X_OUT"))
 (segment (start 125 104.25) (end 125 90.5) (width 0.2) (layer "F.Cu") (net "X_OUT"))
 (segment (start 126.334314 114.25) (end 125.194974 114.25) (width 0.2) (layer "F.Cu") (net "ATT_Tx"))
 (segment (start 125.194974 114.25) (end 121.994974 111.05) (width 0.2) (layer "F.Cu") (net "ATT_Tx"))
 (segment (start 117.732722 111.05) (end 117.217648 111.565074) (width 0.2) (layer "F.Cu") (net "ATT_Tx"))
 (segment (start 126.791851 113.792463) (end 126.334314 114.25) (width 0.2) (layer "F.Cu") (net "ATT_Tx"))
 (segment (start 121.994974 111.05) (end 117.732722 111.05) (width 0.2) (layer "F.Cu") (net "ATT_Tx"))
 (segment (start 125.1 114.65) (end 121.9 111.45) (width 0.2) (layer "F.Cu") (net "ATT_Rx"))
 (segment (start 126.5 114.65) (end 125.1 114.65) (width 0.2) (layer "F.Cu") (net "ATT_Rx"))
 (segment (start 121.9 111.45) (end 119.067574 111.45) (width 0.2) (layer "F.Cu") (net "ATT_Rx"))
 (segment (start 127.074695 114.075305) (end 126.5 114.65) (width 0.2) (layer "F.Cu") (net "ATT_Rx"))
 (segment (start 119.067574 111.45) (end 118.3175 112.200074) (width 0.2) (layer "F.Cu") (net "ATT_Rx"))
 (segment (start 127.357538 114.358147) (end 127 114.715685) (width 0.2) (layer "F.Cu") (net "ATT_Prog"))
 (segment (start 117.6825 115.0325) (end 117.6825 113.299926) (width 0.2) (layer "F.Cu") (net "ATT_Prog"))
 (segment (start 117.680747 115.083073) (end 117.680747 115.034253) (width 0.2) (layer "F.Cu") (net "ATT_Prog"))
 (segment (start 127 117.15) (end 126.4 117.75) (width 0.2) (layer "F.Cu") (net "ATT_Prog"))
 (segment (start 127 114.715685) (end 127 117.15) (width 0.2) (layer "F.Cu") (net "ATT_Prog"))
 (segment (start 117.680747 115.034253) (end 117.6825 115.0325) (width 0.2) (layer "F.Cu") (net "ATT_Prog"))
 (segment (start 126.4 117.75) (end 122.3 117.75) (width 0.2) (layer "F.Cu") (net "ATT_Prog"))
 (segment (start 125.1 111.65) (end 118.3 104.85) (width 0.5) (layer "F.Cu") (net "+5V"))
 (segment (start 137.305179 92.35) (end 137.922592 91.732587) (width 0.5) (layer "F.Cu") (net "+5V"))
 (segment (start 136.6 92.35) (end 137.305179 92.35) (width 0.5) (layer "F.Cu") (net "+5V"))
 (segment (start 111.6 99.45) (end 113.5 97.55) (width 0.5) (layer "F.Cu") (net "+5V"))
 (segment (start 113.7 104.85) (end 111.6 102.75) (width 0.5) (layer "F.Cu") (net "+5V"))
 (segment (start 125.865 115.65) (end 125.915 115.7) (width 0.5) (layer "F.Cu") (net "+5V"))
 (segment (start 113.5 97.55) (end 113.5 95.419005) (width 0.5) (layer "F.Cu") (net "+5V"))
 (segment (start 113.5 95.419005) (end 112.636026 94.555031) (width 0.5) (layer "F.Cu") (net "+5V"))
 (segment (start 111.6 102.75) (end 111.6 99.45) (width 0.5) (layer "F.Cu") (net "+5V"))
 (segment (start 118.3 104.85) (end 113.7 104.85) (width 0.5) (layer "F.Cu") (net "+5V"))
 (segment (start 125.1 115.65) (end 125.865 115.65) (width 0.5) (layer "F.Cu") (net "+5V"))
 (via (at 125.1 111.65) (size 0.8) (drill 0.4) (layers "F.Cu" "B.Cu") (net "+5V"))
 (via (at 125.1 115.65) (size 0.8) (drill 0.4) (layers "F.Cu" "B.Cu") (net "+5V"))
 (via (at 134.9 111.75) (size 0.8) (drill 0.4) (layers "F.Cu" "B.Cu") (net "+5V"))
 (via (at 136.6 92.35) (size 0.8) (drill 0.4) (layers "F.Cu" "B.Cu") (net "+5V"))
 (via (at 134.9 110.15) (size 0.8) (drill 0.4) (layers "F.Cu" "B.Cu") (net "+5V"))
 (segment (start 134.9 110.15) (end 134.9 105.35) (width 1) (layer "B.Cu") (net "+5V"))
 (segment (start 134.9 111.75) (end 134.9 110.15) (width 1) (layer "B.Cu") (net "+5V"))
 (segment (start 116.8 94.95) (end 117.8 94.95) (width 1) (layer "B.Cu") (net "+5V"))
 (segment (start 135.5 96.05) (end 134.4 94.95) (width 1) (layer "B.Cu") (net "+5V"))
 (segment (start 135.5 104.75) (end 135.5 96.05) (width 1) (layer "B.Cu") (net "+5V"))
 (segment (start 117.8 94.95) (end 134.4 94.95) (width 1) (layer "B.Cu") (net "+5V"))
 (segment (start 125.1 111.65) (end 125.1 115.65) (width 0.5) (layer "B.Cu") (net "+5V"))
 (segment (start 112.636026 94.555031) (end 112.641057 94.55) (width 0.5) (layer "B.Cu") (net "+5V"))
 (segment (start 136.6 92.35) (end 134.4 94.55) (width 0.5) (layer "B.Cu") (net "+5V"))
 (segment (start 116.405031 94.555031) (end 116.8 94.95) (width 1) (layer "B.Cu") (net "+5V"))
 (segment (start 134.9 105.35) (end 135.5 104.75) (width 1) (layer "B.Cu") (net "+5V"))
 (segment (start 112.636026 94.555031) (end 116.405031 94.555031) (width 1) (layer "B.Cu") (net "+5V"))
 (segment (start 134.4 94.55) (end 134.4 94.95) (width 0.5) (layer "B.Cu") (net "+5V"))
 (segment (start 123.25 115.7) (end 123.2 115.65) (width 0.25) (layer "F.Cu") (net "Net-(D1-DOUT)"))
 (segment (start 124.085 115.7) (end 123.25 115.7) (width 0.25) (layer "F.Cu") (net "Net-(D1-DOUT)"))
 (via (at 109.6 93.85) (size 0.6) (drill 0.3) (layers "F.Cu" "B.Cu") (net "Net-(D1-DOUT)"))
 (via (at 123.2 115.65) (size 0.6) (drill 0.3) (layers "F.Cu" "B.Cu") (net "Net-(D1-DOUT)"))
 (segment (start 109.2 94.25) (end 109.6 93.85) (width 0.25) (layer "B.Cu") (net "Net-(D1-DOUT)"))
 (segment (start 123.2 115.65) (end 121.9 116.95) (width 0.25) (layer "B.Cu") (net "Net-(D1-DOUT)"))
 (segment (start 121.9 116.95) (end 120.9 116.95) (width 0.25) (layer "B.Cu") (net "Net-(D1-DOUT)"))
 (segment (start 113.885415 107.035415) (end 109.2 102.35) (width 0.25) (layer "B.Cu") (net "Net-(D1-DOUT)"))
 (segment (start 113.885415 112.900128) (end 113.885415 107.035415) (width 0.25) (layer "B.Cu") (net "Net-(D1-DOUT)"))
 (segment (start 109.2 102.35) (end 109.2 94.25) (width 0.25) (layer "B.Cu") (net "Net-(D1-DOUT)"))
 (via (at 112.5 90.95) (size 0.6) (drill 0.3) (layers "F.Cu" "B.Cu") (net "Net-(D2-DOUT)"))
 (via (at 138.3 90.25) (size 0.6) (drill 0.3) (layers "F.Cu" "B.Cu") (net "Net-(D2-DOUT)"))
 (segment (start 112.5 90.95) (end 112.5 90.35) (width 0.25) (layer "B.Cu") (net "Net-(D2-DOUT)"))
 (segment (start 115.4 87.45) (end 135.5 87.45) (width 0.25) (layer "B.Cu") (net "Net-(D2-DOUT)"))
 (segment (start 112.5 90.35) (end 115.4 87.45) (width 0.25) (layer "B.Cu") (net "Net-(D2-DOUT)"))
 (segment (start 135.5 87.45) (end 138.3 90.25) (width 0.25) (layer "B.Cu") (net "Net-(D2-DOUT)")))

